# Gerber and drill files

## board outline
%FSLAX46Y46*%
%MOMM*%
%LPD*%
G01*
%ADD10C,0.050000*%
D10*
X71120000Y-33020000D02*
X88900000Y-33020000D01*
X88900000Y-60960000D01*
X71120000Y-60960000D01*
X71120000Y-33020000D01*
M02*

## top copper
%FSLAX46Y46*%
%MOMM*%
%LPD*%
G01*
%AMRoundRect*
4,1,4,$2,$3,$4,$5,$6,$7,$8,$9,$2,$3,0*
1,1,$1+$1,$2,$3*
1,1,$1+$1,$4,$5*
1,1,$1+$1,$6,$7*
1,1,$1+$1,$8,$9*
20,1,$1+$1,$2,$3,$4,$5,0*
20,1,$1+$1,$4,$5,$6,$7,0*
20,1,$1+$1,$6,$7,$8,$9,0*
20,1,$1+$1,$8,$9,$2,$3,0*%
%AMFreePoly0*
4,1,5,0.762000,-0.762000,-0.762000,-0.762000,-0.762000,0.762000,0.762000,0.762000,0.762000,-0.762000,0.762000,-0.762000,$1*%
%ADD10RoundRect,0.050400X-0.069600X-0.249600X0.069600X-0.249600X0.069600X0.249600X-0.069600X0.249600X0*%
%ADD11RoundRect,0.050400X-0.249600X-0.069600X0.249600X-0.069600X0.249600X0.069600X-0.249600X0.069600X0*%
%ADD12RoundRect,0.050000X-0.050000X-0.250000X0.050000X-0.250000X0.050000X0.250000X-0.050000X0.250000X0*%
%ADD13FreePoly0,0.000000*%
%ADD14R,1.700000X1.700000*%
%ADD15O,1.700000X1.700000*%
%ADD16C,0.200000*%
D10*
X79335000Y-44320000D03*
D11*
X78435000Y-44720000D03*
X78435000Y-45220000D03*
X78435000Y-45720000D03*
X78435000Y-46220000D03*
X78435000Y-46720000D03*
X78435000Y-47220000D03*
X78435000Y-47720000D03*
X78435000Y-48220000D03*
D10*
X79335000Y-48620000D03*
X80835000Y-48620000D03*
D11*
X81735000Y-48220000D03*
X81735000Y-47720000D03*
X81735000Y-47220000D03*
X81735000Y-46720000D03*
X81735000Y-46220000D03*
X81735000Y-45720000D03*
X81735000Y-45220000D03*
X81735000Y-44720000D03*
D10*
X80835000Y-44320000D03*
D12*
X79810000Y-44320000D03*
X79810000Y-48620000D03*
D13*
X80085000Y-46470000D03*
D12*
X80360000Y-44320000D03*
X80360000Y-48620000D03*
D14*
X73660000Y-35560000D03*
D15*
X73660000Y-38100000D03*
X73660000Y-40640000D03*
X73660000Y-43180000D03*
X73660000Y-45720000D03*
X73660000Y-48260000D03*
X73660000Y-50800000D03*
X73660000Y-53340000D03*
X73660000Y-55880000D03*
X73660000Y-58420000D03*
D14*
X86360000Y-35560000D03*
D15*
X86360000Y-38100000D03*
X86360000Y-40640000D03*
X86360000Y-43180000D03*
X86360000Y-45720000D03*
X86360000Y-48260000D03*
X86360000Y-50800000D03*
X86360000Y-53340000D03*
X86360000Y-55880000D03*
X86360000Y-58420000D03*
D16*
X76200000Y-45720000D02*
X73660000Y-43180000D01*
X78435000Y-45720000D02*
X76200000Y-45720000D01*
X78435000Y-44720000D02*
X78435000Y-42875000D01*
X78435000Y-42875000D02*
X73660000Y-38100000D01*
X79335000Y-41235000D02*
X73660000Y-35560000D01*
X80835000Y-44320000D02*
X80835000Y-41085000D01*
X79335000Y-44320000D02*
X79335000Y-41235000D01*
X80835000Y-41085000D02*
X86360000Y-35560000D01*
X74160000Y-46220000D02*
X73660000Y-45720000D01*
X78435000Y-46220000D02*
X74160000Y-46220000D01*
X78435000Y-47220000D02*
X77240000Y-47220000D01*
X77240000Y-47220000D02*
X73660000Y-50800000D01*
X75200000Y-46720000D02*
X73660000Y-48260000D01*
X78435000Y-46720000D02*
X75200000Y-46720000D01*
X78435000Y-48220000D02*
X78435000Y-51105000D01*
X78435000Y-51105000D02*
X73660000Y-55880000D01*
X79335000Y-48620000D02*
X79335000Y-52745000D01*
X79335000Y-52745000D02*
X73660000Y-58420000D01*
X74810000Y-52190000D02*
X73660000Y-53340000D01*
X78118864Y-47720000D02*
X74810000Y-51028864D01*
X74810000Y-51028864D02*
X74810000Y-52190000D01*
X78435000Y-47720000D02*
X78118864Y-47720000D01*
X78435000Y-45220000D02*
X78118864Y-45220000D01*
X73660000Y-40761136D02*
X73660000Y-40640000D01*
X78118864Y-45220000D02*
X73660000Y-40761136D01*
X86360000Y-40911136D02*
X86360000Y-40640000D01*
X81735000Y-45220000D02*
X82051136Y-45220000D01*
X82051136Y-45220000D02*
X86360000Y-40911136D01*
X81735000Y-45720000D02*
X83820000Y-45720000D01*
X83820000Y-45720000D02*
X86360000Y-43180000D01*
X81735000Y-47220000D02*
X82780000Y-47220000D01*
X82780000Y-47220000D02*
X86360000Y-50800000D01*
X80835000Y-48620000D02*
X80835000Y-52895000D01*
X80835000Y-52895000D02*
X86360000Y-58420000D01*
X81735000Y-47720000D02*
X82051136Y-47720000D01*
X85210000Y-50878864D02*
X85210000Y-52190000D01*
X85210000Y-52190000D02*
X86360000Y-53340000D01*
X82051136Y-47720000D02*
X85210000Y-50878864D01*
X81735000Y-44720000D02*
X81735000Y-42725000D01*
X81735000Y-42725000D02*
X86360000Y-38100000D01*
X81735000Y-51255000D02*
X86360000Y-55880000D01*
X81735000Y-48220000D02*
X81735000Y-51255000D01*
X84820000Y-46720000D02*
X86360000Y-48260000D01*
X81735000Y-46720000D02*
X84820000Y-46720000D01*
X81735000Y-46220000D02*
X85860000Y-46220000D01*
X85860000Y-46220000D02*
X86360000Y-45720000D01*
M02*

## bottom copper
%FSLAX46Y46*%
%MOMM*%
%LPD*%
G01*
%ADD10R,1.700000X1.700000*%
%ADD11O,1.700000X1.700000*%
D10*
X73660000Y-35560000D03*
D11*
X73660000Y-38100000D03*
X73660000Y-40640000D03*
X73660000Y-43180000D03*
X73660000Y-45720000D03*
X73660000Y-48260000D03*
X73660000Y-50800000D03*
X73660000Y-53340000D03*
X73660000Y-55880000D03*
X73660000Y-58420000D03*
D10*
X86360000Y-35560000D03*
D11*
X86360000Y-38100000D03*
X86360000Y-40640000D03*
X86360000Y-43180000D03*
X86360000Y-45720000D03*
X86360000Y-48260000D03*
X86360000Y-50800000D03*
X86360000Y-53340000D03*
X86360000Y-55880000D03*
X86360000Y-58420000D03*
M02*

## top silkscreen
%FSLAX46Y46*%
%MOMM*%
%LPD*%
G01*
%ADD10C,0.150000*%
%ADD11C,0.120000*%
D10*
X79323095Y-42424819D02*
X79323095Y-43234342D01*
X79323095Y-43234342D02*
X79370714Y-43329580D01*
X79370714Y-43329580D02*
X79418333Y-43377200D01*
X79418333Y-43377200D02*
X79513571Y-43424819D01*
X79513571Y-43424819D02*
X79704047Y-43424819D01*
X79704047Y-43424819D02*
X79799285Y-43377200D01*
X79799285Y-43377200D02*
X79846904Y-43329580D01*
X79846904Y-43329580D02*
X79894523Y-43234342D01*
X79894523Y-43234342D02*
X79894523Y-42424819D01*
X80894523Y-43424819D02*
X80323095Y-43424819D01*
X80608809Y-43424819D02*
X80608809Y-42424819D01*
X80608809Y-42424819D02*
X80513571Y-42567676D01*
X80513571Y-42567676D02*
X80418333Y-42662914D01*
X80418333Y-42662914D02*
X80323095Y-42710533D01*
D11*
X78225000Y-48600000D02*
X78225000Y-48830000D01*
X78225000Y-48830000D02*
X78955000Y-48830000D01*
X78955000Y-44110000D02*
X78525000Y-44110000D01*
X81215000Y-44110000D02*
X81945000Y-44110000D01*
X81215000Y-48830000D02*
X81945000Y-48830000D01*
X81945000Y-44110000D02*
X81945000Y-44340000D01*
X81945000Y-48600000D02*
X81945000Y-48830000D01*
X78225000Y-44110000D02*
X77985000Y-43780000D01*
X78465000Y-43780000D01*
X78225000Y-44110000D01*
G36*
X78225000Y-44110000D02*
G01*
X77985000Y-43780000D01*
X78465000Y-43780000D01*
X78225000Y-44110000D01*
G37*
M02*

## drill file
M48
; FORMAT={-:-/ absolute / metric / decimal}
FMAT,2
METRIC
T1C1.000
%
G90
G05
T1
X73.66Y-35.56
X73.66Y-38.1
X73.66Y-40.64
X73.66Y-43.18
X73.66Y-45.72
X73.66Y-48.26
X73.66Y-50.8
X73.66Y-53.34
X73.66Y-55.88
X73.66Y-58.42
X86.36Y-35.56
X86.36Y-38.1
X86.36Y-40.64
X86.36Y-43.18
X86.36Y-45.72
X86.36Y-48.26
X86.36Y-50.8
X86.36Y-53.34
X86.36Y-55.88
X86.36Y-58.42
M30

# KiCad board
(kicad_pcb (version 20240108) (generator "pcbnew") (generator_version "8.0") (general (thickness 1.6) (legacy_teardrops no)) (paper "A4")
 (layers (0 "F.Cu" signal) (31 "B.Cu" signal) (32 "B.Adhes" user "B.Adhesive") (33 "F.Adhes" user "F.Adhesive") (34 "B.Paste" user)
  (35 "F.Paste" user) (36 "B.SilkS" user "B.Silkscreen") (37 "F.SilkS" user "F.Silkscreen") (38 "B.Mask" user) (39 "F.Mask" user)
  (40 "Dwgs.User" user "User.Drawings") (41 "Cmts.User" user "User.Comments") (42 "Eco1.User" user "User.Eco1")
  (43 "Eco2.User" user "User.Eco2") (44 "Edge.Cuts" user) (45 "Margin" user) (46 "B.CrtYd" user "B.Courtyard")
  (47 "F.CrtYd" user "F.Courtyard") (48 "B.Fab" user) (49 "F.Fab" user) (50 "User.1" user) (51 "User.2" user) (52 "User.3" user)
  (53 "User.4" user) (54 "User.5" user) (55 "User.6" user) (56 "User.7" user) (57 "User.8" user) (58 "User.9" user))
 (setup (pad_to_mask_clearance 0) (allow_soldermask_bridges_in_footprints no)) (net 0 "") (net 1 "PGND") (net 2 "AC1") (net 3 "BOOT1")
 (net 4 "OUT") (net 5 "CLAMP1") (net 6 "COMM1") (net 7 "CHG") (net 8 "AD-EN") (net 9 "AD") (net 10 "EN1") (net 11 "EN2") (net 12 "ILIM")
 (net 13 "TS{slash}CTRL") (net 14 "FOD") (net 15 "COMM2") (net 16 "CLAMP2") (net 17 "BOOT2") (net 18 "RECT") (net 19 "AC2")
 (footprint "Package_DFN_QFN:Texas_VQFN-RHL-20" (layer "F.Cu") (at 80.085 46.47)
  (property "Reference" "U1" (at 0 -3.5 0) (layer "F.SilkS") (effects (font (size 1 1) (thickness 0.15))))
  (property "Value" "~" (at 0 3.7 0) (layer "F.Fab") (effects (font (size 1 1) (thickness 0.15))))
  (fp_line (start -1.86 2.13) (end -1.86 2.36) (stroke (width 0.12) (type solid)) (layer "F.SilkS"))
  (fp_line (start -1.86 2.36) (end -1.13 2.36) (stroke (width 0.12) (type solid)) (layer "F.SilkS"))
  (fp_line (start -1.13 -2.36) (end -1.56 -2.36) (stroke (width 0.12) (type solid)) (layer "F.SilkS"))
  (fp_line (start 1.13 -2.36) (end 1.86 -2.36) (stroke (width 0.12) (type solid)) (layer "F.SilkS"))
  (fp_line (start 1.13 2.36) (end 1.86 2.36) (stroke (width 0.12) (type solid)) (layer "F.SilkS"))
  (fp_line (start 1.86 -2.36) (end 1.86 -2.13) (stroke (width 0.12) (type solid)) (layer "F.SilkS"))
  (fp_line (start 1.86 2.13) (end 1.86 2.36) (stroke (width 0.12) (type solid)) (layer "F.SilkS"))
  (fp_poly
   (pts (xy -1.86 -2.36) (xy -2.1 -2.69) (xy -1.62 -2.69) (xy -1.86 -2.36)) (stroke (width 0.12) (type solid)) (fill solid)
   (layer "F.SilkS"))
  (pad "" smd rect (at -0.56 -1.05) (size 0.92 0.85) (layers "F.Paste"))
  (pad "" smd rect (at -0.56 0) (size 0.92 0.85) (layers "F.Paste"))
  (pad "" smd rect (at -0.56 1.05) (size 0.92 0.85) (layers "F.Paste"))
  (pad "" smd rect (at 0 -1.8) (size 0.75 0.25) (layers "F.Paste"))
  (pad "" smd rect (at 0 1.8) (size 0.75 0.25) (layers "F.Paste"))
  (pad "" smd rect (at 0.56 -1.05) (size 0.92 0.85) (layers "F.Paste"))
  (pad "" smd rect (at 0.56 0) (size 0.92 0.85) (layers "F.Paste"))
  (pad "" smd rect (at 0.56 1.05) (size 0.92 0.85) (layers "F.Paste"))
  (pad "1" smd roundrect (at -0.75 -2.15) (size 0.24 0.6) (layers "F.Cu" "F.Paste" "F.Mask") (roundrect_rratio 0.21) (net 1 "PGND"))
  (pad "2" smd roundrect (at -1.65 -1.75) (size 0.6 0.24) (layers "F.Cu" "F.Paste" "F.Mask") (roundrect_rratio 0.21) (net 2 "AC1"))
  (pad "3" smd roundrect (at -1.65 -1.25) (size 0.6 0.24) (layers "F.Cu" "F.Paste" "F.Mask") (roundrect_rratio 0.21) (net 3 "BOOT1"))
  (pad "4" smd roundrect (at -1.65 -0.75) (size 0.6 0.24) (layers "F.Cu" "F.Paste" "F.Mask") (roundrect_rratio 0.21) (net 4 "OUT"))
  (pad "5" smd roundrect (at -1.65 -0.25) (size 0.6 0.24) (layers "F.Cu" "F.Paste" "F.Mask") (roundrect_rratio 0.21) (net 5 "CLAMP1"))
  (pad "6" smd roundrect (at -1.65 0.25) (size 0.6 0.24) (layers "F.Cu" "F.Paste" "F.Mask") (roundrect_rratio 0.21) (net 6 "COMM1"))
  (pad "7" smd roundrect (at -1.65 0.75) (size 0.6 0.24) (layers "F.Cu" "F.Paste" "F.Mask") (roundrect_rratio 0.21) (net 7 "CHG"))
  (pad "8" smd roundrect (at -1.65 1.25) (size 0.6 0.24) (layers "F.Cu" "F.Paste" "F.Mask") (roundrect_rratio 0.21) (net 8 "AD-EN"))
  (pad "9" smd roundrect (at -1.65 1.75) (size 0.6 0.24) (layers "F.Cu" "F.Paste" "F.Mask") (roundrect_rratio 0.21) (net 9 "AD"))
  (pad "10" smd roundrect (at -0.75 2.15) (size 0.24 0.6) (layers "F.Cu" "F.Paste" "F.Mask") (roundrect_rratio 0.21) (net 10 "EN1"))
  (pad "11" smd roundrect (at 0.75 2.15) (size 0.24 0.6) (layers "F.Cu" "F.Paste" "F.Mask") (roundrect_rratio 0.21) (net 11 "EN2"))
  (pad "12" smd roundrect (at 1.65 1.75) (size 0.6 0.24) (layers "F.Cu" "F.Paste" "F.Mask") (roundrect_rratio 0.21) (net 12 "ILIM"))
  (pad "13" smd roundrect (at 1.65 1.25) (size 0.6 0.24) (layers "F.Cu" "F.Paste" "F.Mask") (roundrect_rratio 0.21) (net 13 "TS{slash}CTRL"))
  (pad "14" smd roundrect (at 1.65 0.75) (size 0.6 0.24) (layers "F.Cu" "F.Paste" "F.Mask") (roundrect_rratio 0.21) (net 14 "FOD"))
  (pad "15" smd roundrect (at 1.65 0.25) (size 0.6 0.24) (layers "F.Cu" "F.Paste" "F.Mask") (roundrect_rratio 0.21) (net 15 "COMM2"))
  (pad "16" smd roundrect (at 1.65 -0.25) (size 0.6 0.24) (layers "F.Cu" "F.Paste" "F.Mask") (roundrect_rratio 0.21) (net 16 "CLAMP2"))
  (pad "17" smd roundrect (at 1.65 -0.75) (size 0.6 0.24) (layers "F.Cu" "F.Paste" "F.Mask") (roundrect_rratio 0.21) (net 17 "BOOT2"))
  (pad "18" smd roundrect (at 1.65 -1.25) (size 0.6 0.24) (layers "F.Cu" "F.Paste" "F.Mask") (roundrect_rratio 0.21) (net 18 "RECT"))
  (pad "19" smd roundrect (at 1.65 -1.75) (size 0.6 0.24) (layers "F.Cu" "F.Paste" "F.Mask") (roundrect_rratio 0.21) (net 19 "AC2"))
  (pad "20" smd roundrect (at 0.75 -2.15) (size 0.24 0.6) (layers "F.Cu" "F.Paste" "F.Mask") (roundrect_rratio 0.21) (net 1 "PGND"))
  (pad "21" smd roundrect (at -0.275 -2.15) (size 0.2 0.6) (layers "F.Cu" "F.Paste" "F.Mask") (roundrect_rratio 0.25))
  (pad "21" smd roundrect (at -0.275 2.15) (size 0.2 0.6) (layers "F.Cu" "F.Paste" "F.Mask") (roundrect_rratio 0.25))
  (pad "21" smd custom (at 0 0) (size 1.524 1.524) (layers "F.Cu" "F.Mask") (zone_connect 0) (thermal_bridge_angle 45)
   (options (clearance outline) (anchor rect)) (primitives))
  (pad "21" smd roundrect (at 0.275 -2.15) (size 0.2 0.6) (layers "F.Cu" "F.Paste" "F.Mask") (roundrect_rratio 0.25))
  (pad "21" smd roundrect (at 0.275 2.15) (size 0.2 0.6) (layers "F.Cu" "F.Paste" "F.Mask") (roundrect_rratio 0.25)))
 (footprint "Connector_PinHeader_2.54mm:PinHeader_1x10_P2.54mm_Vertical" (layer "B.Cu") (at 73.66 35.56 180)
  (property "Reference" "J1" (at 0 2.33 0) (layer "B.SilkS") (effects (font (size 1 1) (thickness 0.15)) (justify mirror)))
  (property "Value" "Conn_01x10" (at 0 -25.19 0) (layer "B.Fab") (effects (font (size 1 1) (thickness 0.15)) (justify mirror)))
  (pad "1" thru_hole rect (at 0 0 180) (size 1.7 1.7) (drill 1) (layers "*.Cu" "*.Mask") (remove_unused_layers no) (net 1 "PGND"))
  (pad "2" thru_hole oval (at 0 -2.54 180) (size 1.7 1.7) (drill 1) (layers "*.Cu" "*.Mask") (remove_unused_layers no) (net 2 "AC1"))
  (pad "3" thru_hole oval (at 0 -5.08 180) (size 1.7 1.7) (drill 1) (layers "*.Cu" "*.Mask") (remove_unused_layers no) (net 3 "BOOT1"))
  (pad "4" thru_hole oval (at 0 -7.62 180) (size 1.7 1.7) (drill 1) (layers "*.Cu" "*.Mask") (remove_unused_layers no) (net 4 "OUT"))
  (pad "5" thru_hole oval (at 0 -10.16 180) (size 1.7 1.7) (drill 1) (layers "*.Cu" "*.Mask") (remove_unused_layers no) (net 5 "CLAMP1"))
  (pad "6" thru_hole oval (at 0 -12.7 180) (size 1.7 1.7) (drill 1) (layers "*.Cu" "*.Mask") (remove_unused_layers no) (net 6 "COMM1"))
  (pad "7" thru_hole oval (at 0 -15.24 180) (size 1.7 1.7) (drill 1) (layers "*.Cu" "*.Mask") (remove_unused_layers no) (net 7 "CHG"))
  (pad "8" thru_hole oval (at 0 -17.78 180) (size 1.7 1.7) (drill 1) (layers "*.Cu" "*.Mask") (remove_unused_layers no) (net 8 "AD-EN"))
  (pad "9" thru_hole oval (at 0 -20.32 180) (size 1.7 1.7) (drill 1) (layers "*.Cu" "*.Mask") (remove_unused_layers no) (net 9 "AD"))
  (pad "10" thru_hole oval (at 0 -22.86 180) (size 1.7 1.7) (drill 1) (layers "*.Cu" "*.Mask") (remove_unused_layers no) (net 10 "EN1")))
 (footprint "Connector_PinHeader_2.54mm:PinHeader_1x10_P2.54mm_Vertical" (layer "B.Cu") (at 86.36 35.56 180)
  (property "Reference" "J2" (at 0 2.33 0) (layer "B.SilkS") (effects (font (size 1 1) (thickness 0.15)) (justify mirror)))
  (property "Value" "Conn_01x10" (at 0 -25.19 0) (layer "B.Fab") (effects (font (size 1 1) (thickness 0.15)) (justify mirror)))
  (pad "1" thru_hole rect (at 0 0 180) (size 1.7 1.7) (drill 1) (layers "*.Cu" "*.Mask") (remove_unused_layers no) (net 1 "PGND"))
  (pad "2" thru_hole oval (at 0 -2.54 180) (size 1.7 1.7) (drill 1) (layers "*.Cu" "*.Mask") (remove_unused_layers no) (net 19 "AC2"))
  (pad "3" thru_hole oval (at 0 -5.08 180) (size 1.7 1.7) (drill 1) (layers "*.Cu" "*.Mask") (remove_unused_layers no) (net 18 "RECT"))
  (pad "4" thru_hole oval (at 0 -7.62 180) (size 1.7 1.7) (drill 1) (layers "*.Cu" "*.Mask") (remove_unused_layers no) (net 17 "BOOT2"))
  (pad "5" thru_hole oval (at 0 -10.16 180) (size 1.7 1.7) (drill 1) (layers "*.Cu" "*.Mask") (remove_unused_layers no) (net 16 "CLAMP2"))
  (pad "6" thru_hole oval (at 0 -12.7 180) (size 1.7 1.7) (drill 1) (layers "*.Cu" "*.Mask") (remove_unused_layers no) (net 15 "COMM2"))
  (pad "7" thru_hole oval (at 0 -15.24 180) (size 1.7 1.7) (drill 1) (layers "*.Cu" "*.Mask") (remove_unused_layers no) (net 14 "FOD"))
  (pad "8" thru_hole oval (at 0 -17.78 180) (size 1.7 1.7) (drill 1) (layers "*.Cu" "*.Mask") (remove_unused_layers no)
   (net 13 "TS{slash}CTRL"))
  (pad "9" thru_hole oval (at 0 -20.32 180) (size 1.7 1.7) (drill 1) (layers "*.Cu" "*.Mask") (remove_unused_layers no) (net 12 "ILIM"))
  (pad "10" thru_hole oval (at 0 -22.86 180) (size 1.7 1.7) (drill 1) (layers "*.Cu" "*.Mask") (remove_unused_layers no) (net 11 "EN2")))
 (gr_rect (start 71.12 33.02) (end 88.9 60.96) (stroke (width 0.05) (type default)) (fill none) (layer "Edge.Cuts"))
 (segment (start 76.2 45.72) (end 73.66 43.18) (width 0.2) (layer "F.Cu") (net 4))
 (segment (start 78.435 45.72) (end 76.2 45.72) (width 0.2) (layer "F.Cu") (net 4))
 (segment (start 78.435 44.72) (end 78.435 42.875) (width 0.2) (layer "F.Cu") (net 2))
 (segment (start 78.435 42.875) (end 73.66 38.1) (width 0.2) (layer "F.Cu") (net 2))
 (segment (start 79.335 41.235) (end 73.66 35.56) (width 0.2) (layer "F.Cu") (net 1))
 (segment (start 80.835 44.32) (end 80.835 41.085) (width 0.2) (layer "F.Cu") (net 1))
 (segment (start 79.335 44.32) (end 79.335 41.235) (width 0.2) (layer "F.Cu") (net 1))
 (segment (start 80.835 41.085) (end 86.36 35.56) (width 0.2) (layer "F.Cu") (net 1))
 (segment (start 74.16 46.22) (end 73.66 45.72) (width 0.2) (layer "F.Cu") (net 5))
 (segment (start 78.435 46.22) (end 74.16 46.22) (width 0.2) (layer "F.Cu") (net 5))
 (segment (start 78.435 47.22) (end 77.24 47.22) (width 0.2) (layer "F.Cu") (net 7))
 (segment (start 77.24 47.22) (end 73.66 50.8) (width 0.2) (layer "F.Cu") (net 7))
 (segment (start 75.2 46.72) (end 73.66 48.26) (width 0.2) (layer "F.Cu") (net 6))
 (segment (start 78.435 46.72) (end 75.2 46.72) (width 0.2) (layer "F.Cu") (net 6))
 (segment (start 78.435 48.22) (end 78.435 51.105) (width 0.2) (layer "F.Cu") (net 9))
 (segment (start 78.435 51.105) (end 73.66 55.88) (width 0.2) (layer "F.Cu") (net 9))
 (segment (start 79.335 48.62) (end 79.335 52.745) (width 0.2) (layer "F.Cu") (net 10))
 (segment (start 79.335 52.745) (end 73.66 58.42) (width 0.2) (layer "F.Cu") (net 10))
 (segment (start 74.81 52.19) (end 73.66 53.34) (width 0.2) (layer "F.Cu") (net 8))
 (segment (start 78.118864 47.72) (end 74.81 51.028864) (width 0.2) (layer "F.Cu") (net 8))
 (segment (start 74.81 51.028864) (end 74.81 52.19) (width 0.2) (layer "F.Cu") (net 8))
 (segment (start 78.435 47.72) (end 78.118864 47.72) (width 0.2) (layer "F.Cu") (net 8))
 (segment (start 78.435 45.22) (end 78.118864 45.22) (width 0.2) (layer "F.Cu") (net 3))
 (segment (start 73.66 40.761136) (end 73.66 40.64) (width 0.2) (layer "F.Cu") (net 3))
 (segment (start 78.118864 45.22) (end 73.66 40.761136) (width 0.2) (layer "F.Cu") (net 3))
 (segment (start 86.36 40.911136) (end 86.36 40.64) (width 0.2) (layer "F.Cu") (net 18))
 (segment (start 81.735 45.22) (end 82.051136 45.22) (width 0.2) (layer "F.Cu") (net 18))
 (segment (start 82.051136 45.22) (end 86.36 40.911136) (width 0.2) (layer "F.Cu") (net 18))
 (segment (start 81.735 45.72) (end 83.82 45.72) (width 0.2) (layer "F.Cu") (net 17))
 (segment (start 83.82 45.72) (end 86.36 43.18) (width 0.2) (layer "F.Cu") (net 17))
 (segment (start 81.735 47.22) (end 82.78 47.22) (width 0.2) (layer "F.Cu") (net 14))
 (segment (start 82.78 47.22) (end 86.36 50.8) (width 0.2) (layer "F.Cu") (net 14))
 (segment (start 80.835 48.62) (end 80.835 52.895) (width 0.2) (layer "F.Cu") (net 11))
 (segment (start 80.835 52.895) (end 86.36 58.42) (width 0.2) (layer "F.Cu") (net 11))
 (segment (start 81.735 47.72) (end 82.051136 47.72) (width 0.2) (layer "F.Cu") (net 13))
 (segment (start 85.21 50.878864) (end 85.21 52.19) (width 0.2) (layer "F.Cu") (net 13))
 (segment (start 85.21 52.19) (end 86.36 53.34) (width 0.2) (layer "F.Cu") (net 13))
 (segment (start 82.051136 47.72) (end 85.21 50.878864) (width 0.2) (layer "F.Cu") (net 13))
 (segment (start 81.735 44.72) (end 81.735 42.725) (width 0.2) (layer "F.Cu") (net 19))
 (segment (start 81.735 42.725) (end 86.36 38.1) (width 0.2) (layer "F.Cu") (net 19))
 (segment (start 81.735 51.255) (end 86.36 55.88) (width 0.2) (layer "F.Cu") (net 12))
 (segment (start 81.735 48.22) (end 81.735 51.255) (width 0.2) (layer "F.Cu") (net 12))
 (segment (start 84.82 46.72) (end 86.36 48.26) (width 0.2) (layer "F.Cu") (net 15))
 (segment (start 81.735 46.72) (end 84.82 46.72) (width 0.2) (layer "F.Cu") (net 15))
 (segment (start 81.735 46.22) (end 85.86 46.22) (width 0.2) (layer "F.Cu") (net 16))
 (segment (start 85.86 46.22) (end 86.36 45.72) (width 0.2) (layer "F.Cu") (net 16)))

